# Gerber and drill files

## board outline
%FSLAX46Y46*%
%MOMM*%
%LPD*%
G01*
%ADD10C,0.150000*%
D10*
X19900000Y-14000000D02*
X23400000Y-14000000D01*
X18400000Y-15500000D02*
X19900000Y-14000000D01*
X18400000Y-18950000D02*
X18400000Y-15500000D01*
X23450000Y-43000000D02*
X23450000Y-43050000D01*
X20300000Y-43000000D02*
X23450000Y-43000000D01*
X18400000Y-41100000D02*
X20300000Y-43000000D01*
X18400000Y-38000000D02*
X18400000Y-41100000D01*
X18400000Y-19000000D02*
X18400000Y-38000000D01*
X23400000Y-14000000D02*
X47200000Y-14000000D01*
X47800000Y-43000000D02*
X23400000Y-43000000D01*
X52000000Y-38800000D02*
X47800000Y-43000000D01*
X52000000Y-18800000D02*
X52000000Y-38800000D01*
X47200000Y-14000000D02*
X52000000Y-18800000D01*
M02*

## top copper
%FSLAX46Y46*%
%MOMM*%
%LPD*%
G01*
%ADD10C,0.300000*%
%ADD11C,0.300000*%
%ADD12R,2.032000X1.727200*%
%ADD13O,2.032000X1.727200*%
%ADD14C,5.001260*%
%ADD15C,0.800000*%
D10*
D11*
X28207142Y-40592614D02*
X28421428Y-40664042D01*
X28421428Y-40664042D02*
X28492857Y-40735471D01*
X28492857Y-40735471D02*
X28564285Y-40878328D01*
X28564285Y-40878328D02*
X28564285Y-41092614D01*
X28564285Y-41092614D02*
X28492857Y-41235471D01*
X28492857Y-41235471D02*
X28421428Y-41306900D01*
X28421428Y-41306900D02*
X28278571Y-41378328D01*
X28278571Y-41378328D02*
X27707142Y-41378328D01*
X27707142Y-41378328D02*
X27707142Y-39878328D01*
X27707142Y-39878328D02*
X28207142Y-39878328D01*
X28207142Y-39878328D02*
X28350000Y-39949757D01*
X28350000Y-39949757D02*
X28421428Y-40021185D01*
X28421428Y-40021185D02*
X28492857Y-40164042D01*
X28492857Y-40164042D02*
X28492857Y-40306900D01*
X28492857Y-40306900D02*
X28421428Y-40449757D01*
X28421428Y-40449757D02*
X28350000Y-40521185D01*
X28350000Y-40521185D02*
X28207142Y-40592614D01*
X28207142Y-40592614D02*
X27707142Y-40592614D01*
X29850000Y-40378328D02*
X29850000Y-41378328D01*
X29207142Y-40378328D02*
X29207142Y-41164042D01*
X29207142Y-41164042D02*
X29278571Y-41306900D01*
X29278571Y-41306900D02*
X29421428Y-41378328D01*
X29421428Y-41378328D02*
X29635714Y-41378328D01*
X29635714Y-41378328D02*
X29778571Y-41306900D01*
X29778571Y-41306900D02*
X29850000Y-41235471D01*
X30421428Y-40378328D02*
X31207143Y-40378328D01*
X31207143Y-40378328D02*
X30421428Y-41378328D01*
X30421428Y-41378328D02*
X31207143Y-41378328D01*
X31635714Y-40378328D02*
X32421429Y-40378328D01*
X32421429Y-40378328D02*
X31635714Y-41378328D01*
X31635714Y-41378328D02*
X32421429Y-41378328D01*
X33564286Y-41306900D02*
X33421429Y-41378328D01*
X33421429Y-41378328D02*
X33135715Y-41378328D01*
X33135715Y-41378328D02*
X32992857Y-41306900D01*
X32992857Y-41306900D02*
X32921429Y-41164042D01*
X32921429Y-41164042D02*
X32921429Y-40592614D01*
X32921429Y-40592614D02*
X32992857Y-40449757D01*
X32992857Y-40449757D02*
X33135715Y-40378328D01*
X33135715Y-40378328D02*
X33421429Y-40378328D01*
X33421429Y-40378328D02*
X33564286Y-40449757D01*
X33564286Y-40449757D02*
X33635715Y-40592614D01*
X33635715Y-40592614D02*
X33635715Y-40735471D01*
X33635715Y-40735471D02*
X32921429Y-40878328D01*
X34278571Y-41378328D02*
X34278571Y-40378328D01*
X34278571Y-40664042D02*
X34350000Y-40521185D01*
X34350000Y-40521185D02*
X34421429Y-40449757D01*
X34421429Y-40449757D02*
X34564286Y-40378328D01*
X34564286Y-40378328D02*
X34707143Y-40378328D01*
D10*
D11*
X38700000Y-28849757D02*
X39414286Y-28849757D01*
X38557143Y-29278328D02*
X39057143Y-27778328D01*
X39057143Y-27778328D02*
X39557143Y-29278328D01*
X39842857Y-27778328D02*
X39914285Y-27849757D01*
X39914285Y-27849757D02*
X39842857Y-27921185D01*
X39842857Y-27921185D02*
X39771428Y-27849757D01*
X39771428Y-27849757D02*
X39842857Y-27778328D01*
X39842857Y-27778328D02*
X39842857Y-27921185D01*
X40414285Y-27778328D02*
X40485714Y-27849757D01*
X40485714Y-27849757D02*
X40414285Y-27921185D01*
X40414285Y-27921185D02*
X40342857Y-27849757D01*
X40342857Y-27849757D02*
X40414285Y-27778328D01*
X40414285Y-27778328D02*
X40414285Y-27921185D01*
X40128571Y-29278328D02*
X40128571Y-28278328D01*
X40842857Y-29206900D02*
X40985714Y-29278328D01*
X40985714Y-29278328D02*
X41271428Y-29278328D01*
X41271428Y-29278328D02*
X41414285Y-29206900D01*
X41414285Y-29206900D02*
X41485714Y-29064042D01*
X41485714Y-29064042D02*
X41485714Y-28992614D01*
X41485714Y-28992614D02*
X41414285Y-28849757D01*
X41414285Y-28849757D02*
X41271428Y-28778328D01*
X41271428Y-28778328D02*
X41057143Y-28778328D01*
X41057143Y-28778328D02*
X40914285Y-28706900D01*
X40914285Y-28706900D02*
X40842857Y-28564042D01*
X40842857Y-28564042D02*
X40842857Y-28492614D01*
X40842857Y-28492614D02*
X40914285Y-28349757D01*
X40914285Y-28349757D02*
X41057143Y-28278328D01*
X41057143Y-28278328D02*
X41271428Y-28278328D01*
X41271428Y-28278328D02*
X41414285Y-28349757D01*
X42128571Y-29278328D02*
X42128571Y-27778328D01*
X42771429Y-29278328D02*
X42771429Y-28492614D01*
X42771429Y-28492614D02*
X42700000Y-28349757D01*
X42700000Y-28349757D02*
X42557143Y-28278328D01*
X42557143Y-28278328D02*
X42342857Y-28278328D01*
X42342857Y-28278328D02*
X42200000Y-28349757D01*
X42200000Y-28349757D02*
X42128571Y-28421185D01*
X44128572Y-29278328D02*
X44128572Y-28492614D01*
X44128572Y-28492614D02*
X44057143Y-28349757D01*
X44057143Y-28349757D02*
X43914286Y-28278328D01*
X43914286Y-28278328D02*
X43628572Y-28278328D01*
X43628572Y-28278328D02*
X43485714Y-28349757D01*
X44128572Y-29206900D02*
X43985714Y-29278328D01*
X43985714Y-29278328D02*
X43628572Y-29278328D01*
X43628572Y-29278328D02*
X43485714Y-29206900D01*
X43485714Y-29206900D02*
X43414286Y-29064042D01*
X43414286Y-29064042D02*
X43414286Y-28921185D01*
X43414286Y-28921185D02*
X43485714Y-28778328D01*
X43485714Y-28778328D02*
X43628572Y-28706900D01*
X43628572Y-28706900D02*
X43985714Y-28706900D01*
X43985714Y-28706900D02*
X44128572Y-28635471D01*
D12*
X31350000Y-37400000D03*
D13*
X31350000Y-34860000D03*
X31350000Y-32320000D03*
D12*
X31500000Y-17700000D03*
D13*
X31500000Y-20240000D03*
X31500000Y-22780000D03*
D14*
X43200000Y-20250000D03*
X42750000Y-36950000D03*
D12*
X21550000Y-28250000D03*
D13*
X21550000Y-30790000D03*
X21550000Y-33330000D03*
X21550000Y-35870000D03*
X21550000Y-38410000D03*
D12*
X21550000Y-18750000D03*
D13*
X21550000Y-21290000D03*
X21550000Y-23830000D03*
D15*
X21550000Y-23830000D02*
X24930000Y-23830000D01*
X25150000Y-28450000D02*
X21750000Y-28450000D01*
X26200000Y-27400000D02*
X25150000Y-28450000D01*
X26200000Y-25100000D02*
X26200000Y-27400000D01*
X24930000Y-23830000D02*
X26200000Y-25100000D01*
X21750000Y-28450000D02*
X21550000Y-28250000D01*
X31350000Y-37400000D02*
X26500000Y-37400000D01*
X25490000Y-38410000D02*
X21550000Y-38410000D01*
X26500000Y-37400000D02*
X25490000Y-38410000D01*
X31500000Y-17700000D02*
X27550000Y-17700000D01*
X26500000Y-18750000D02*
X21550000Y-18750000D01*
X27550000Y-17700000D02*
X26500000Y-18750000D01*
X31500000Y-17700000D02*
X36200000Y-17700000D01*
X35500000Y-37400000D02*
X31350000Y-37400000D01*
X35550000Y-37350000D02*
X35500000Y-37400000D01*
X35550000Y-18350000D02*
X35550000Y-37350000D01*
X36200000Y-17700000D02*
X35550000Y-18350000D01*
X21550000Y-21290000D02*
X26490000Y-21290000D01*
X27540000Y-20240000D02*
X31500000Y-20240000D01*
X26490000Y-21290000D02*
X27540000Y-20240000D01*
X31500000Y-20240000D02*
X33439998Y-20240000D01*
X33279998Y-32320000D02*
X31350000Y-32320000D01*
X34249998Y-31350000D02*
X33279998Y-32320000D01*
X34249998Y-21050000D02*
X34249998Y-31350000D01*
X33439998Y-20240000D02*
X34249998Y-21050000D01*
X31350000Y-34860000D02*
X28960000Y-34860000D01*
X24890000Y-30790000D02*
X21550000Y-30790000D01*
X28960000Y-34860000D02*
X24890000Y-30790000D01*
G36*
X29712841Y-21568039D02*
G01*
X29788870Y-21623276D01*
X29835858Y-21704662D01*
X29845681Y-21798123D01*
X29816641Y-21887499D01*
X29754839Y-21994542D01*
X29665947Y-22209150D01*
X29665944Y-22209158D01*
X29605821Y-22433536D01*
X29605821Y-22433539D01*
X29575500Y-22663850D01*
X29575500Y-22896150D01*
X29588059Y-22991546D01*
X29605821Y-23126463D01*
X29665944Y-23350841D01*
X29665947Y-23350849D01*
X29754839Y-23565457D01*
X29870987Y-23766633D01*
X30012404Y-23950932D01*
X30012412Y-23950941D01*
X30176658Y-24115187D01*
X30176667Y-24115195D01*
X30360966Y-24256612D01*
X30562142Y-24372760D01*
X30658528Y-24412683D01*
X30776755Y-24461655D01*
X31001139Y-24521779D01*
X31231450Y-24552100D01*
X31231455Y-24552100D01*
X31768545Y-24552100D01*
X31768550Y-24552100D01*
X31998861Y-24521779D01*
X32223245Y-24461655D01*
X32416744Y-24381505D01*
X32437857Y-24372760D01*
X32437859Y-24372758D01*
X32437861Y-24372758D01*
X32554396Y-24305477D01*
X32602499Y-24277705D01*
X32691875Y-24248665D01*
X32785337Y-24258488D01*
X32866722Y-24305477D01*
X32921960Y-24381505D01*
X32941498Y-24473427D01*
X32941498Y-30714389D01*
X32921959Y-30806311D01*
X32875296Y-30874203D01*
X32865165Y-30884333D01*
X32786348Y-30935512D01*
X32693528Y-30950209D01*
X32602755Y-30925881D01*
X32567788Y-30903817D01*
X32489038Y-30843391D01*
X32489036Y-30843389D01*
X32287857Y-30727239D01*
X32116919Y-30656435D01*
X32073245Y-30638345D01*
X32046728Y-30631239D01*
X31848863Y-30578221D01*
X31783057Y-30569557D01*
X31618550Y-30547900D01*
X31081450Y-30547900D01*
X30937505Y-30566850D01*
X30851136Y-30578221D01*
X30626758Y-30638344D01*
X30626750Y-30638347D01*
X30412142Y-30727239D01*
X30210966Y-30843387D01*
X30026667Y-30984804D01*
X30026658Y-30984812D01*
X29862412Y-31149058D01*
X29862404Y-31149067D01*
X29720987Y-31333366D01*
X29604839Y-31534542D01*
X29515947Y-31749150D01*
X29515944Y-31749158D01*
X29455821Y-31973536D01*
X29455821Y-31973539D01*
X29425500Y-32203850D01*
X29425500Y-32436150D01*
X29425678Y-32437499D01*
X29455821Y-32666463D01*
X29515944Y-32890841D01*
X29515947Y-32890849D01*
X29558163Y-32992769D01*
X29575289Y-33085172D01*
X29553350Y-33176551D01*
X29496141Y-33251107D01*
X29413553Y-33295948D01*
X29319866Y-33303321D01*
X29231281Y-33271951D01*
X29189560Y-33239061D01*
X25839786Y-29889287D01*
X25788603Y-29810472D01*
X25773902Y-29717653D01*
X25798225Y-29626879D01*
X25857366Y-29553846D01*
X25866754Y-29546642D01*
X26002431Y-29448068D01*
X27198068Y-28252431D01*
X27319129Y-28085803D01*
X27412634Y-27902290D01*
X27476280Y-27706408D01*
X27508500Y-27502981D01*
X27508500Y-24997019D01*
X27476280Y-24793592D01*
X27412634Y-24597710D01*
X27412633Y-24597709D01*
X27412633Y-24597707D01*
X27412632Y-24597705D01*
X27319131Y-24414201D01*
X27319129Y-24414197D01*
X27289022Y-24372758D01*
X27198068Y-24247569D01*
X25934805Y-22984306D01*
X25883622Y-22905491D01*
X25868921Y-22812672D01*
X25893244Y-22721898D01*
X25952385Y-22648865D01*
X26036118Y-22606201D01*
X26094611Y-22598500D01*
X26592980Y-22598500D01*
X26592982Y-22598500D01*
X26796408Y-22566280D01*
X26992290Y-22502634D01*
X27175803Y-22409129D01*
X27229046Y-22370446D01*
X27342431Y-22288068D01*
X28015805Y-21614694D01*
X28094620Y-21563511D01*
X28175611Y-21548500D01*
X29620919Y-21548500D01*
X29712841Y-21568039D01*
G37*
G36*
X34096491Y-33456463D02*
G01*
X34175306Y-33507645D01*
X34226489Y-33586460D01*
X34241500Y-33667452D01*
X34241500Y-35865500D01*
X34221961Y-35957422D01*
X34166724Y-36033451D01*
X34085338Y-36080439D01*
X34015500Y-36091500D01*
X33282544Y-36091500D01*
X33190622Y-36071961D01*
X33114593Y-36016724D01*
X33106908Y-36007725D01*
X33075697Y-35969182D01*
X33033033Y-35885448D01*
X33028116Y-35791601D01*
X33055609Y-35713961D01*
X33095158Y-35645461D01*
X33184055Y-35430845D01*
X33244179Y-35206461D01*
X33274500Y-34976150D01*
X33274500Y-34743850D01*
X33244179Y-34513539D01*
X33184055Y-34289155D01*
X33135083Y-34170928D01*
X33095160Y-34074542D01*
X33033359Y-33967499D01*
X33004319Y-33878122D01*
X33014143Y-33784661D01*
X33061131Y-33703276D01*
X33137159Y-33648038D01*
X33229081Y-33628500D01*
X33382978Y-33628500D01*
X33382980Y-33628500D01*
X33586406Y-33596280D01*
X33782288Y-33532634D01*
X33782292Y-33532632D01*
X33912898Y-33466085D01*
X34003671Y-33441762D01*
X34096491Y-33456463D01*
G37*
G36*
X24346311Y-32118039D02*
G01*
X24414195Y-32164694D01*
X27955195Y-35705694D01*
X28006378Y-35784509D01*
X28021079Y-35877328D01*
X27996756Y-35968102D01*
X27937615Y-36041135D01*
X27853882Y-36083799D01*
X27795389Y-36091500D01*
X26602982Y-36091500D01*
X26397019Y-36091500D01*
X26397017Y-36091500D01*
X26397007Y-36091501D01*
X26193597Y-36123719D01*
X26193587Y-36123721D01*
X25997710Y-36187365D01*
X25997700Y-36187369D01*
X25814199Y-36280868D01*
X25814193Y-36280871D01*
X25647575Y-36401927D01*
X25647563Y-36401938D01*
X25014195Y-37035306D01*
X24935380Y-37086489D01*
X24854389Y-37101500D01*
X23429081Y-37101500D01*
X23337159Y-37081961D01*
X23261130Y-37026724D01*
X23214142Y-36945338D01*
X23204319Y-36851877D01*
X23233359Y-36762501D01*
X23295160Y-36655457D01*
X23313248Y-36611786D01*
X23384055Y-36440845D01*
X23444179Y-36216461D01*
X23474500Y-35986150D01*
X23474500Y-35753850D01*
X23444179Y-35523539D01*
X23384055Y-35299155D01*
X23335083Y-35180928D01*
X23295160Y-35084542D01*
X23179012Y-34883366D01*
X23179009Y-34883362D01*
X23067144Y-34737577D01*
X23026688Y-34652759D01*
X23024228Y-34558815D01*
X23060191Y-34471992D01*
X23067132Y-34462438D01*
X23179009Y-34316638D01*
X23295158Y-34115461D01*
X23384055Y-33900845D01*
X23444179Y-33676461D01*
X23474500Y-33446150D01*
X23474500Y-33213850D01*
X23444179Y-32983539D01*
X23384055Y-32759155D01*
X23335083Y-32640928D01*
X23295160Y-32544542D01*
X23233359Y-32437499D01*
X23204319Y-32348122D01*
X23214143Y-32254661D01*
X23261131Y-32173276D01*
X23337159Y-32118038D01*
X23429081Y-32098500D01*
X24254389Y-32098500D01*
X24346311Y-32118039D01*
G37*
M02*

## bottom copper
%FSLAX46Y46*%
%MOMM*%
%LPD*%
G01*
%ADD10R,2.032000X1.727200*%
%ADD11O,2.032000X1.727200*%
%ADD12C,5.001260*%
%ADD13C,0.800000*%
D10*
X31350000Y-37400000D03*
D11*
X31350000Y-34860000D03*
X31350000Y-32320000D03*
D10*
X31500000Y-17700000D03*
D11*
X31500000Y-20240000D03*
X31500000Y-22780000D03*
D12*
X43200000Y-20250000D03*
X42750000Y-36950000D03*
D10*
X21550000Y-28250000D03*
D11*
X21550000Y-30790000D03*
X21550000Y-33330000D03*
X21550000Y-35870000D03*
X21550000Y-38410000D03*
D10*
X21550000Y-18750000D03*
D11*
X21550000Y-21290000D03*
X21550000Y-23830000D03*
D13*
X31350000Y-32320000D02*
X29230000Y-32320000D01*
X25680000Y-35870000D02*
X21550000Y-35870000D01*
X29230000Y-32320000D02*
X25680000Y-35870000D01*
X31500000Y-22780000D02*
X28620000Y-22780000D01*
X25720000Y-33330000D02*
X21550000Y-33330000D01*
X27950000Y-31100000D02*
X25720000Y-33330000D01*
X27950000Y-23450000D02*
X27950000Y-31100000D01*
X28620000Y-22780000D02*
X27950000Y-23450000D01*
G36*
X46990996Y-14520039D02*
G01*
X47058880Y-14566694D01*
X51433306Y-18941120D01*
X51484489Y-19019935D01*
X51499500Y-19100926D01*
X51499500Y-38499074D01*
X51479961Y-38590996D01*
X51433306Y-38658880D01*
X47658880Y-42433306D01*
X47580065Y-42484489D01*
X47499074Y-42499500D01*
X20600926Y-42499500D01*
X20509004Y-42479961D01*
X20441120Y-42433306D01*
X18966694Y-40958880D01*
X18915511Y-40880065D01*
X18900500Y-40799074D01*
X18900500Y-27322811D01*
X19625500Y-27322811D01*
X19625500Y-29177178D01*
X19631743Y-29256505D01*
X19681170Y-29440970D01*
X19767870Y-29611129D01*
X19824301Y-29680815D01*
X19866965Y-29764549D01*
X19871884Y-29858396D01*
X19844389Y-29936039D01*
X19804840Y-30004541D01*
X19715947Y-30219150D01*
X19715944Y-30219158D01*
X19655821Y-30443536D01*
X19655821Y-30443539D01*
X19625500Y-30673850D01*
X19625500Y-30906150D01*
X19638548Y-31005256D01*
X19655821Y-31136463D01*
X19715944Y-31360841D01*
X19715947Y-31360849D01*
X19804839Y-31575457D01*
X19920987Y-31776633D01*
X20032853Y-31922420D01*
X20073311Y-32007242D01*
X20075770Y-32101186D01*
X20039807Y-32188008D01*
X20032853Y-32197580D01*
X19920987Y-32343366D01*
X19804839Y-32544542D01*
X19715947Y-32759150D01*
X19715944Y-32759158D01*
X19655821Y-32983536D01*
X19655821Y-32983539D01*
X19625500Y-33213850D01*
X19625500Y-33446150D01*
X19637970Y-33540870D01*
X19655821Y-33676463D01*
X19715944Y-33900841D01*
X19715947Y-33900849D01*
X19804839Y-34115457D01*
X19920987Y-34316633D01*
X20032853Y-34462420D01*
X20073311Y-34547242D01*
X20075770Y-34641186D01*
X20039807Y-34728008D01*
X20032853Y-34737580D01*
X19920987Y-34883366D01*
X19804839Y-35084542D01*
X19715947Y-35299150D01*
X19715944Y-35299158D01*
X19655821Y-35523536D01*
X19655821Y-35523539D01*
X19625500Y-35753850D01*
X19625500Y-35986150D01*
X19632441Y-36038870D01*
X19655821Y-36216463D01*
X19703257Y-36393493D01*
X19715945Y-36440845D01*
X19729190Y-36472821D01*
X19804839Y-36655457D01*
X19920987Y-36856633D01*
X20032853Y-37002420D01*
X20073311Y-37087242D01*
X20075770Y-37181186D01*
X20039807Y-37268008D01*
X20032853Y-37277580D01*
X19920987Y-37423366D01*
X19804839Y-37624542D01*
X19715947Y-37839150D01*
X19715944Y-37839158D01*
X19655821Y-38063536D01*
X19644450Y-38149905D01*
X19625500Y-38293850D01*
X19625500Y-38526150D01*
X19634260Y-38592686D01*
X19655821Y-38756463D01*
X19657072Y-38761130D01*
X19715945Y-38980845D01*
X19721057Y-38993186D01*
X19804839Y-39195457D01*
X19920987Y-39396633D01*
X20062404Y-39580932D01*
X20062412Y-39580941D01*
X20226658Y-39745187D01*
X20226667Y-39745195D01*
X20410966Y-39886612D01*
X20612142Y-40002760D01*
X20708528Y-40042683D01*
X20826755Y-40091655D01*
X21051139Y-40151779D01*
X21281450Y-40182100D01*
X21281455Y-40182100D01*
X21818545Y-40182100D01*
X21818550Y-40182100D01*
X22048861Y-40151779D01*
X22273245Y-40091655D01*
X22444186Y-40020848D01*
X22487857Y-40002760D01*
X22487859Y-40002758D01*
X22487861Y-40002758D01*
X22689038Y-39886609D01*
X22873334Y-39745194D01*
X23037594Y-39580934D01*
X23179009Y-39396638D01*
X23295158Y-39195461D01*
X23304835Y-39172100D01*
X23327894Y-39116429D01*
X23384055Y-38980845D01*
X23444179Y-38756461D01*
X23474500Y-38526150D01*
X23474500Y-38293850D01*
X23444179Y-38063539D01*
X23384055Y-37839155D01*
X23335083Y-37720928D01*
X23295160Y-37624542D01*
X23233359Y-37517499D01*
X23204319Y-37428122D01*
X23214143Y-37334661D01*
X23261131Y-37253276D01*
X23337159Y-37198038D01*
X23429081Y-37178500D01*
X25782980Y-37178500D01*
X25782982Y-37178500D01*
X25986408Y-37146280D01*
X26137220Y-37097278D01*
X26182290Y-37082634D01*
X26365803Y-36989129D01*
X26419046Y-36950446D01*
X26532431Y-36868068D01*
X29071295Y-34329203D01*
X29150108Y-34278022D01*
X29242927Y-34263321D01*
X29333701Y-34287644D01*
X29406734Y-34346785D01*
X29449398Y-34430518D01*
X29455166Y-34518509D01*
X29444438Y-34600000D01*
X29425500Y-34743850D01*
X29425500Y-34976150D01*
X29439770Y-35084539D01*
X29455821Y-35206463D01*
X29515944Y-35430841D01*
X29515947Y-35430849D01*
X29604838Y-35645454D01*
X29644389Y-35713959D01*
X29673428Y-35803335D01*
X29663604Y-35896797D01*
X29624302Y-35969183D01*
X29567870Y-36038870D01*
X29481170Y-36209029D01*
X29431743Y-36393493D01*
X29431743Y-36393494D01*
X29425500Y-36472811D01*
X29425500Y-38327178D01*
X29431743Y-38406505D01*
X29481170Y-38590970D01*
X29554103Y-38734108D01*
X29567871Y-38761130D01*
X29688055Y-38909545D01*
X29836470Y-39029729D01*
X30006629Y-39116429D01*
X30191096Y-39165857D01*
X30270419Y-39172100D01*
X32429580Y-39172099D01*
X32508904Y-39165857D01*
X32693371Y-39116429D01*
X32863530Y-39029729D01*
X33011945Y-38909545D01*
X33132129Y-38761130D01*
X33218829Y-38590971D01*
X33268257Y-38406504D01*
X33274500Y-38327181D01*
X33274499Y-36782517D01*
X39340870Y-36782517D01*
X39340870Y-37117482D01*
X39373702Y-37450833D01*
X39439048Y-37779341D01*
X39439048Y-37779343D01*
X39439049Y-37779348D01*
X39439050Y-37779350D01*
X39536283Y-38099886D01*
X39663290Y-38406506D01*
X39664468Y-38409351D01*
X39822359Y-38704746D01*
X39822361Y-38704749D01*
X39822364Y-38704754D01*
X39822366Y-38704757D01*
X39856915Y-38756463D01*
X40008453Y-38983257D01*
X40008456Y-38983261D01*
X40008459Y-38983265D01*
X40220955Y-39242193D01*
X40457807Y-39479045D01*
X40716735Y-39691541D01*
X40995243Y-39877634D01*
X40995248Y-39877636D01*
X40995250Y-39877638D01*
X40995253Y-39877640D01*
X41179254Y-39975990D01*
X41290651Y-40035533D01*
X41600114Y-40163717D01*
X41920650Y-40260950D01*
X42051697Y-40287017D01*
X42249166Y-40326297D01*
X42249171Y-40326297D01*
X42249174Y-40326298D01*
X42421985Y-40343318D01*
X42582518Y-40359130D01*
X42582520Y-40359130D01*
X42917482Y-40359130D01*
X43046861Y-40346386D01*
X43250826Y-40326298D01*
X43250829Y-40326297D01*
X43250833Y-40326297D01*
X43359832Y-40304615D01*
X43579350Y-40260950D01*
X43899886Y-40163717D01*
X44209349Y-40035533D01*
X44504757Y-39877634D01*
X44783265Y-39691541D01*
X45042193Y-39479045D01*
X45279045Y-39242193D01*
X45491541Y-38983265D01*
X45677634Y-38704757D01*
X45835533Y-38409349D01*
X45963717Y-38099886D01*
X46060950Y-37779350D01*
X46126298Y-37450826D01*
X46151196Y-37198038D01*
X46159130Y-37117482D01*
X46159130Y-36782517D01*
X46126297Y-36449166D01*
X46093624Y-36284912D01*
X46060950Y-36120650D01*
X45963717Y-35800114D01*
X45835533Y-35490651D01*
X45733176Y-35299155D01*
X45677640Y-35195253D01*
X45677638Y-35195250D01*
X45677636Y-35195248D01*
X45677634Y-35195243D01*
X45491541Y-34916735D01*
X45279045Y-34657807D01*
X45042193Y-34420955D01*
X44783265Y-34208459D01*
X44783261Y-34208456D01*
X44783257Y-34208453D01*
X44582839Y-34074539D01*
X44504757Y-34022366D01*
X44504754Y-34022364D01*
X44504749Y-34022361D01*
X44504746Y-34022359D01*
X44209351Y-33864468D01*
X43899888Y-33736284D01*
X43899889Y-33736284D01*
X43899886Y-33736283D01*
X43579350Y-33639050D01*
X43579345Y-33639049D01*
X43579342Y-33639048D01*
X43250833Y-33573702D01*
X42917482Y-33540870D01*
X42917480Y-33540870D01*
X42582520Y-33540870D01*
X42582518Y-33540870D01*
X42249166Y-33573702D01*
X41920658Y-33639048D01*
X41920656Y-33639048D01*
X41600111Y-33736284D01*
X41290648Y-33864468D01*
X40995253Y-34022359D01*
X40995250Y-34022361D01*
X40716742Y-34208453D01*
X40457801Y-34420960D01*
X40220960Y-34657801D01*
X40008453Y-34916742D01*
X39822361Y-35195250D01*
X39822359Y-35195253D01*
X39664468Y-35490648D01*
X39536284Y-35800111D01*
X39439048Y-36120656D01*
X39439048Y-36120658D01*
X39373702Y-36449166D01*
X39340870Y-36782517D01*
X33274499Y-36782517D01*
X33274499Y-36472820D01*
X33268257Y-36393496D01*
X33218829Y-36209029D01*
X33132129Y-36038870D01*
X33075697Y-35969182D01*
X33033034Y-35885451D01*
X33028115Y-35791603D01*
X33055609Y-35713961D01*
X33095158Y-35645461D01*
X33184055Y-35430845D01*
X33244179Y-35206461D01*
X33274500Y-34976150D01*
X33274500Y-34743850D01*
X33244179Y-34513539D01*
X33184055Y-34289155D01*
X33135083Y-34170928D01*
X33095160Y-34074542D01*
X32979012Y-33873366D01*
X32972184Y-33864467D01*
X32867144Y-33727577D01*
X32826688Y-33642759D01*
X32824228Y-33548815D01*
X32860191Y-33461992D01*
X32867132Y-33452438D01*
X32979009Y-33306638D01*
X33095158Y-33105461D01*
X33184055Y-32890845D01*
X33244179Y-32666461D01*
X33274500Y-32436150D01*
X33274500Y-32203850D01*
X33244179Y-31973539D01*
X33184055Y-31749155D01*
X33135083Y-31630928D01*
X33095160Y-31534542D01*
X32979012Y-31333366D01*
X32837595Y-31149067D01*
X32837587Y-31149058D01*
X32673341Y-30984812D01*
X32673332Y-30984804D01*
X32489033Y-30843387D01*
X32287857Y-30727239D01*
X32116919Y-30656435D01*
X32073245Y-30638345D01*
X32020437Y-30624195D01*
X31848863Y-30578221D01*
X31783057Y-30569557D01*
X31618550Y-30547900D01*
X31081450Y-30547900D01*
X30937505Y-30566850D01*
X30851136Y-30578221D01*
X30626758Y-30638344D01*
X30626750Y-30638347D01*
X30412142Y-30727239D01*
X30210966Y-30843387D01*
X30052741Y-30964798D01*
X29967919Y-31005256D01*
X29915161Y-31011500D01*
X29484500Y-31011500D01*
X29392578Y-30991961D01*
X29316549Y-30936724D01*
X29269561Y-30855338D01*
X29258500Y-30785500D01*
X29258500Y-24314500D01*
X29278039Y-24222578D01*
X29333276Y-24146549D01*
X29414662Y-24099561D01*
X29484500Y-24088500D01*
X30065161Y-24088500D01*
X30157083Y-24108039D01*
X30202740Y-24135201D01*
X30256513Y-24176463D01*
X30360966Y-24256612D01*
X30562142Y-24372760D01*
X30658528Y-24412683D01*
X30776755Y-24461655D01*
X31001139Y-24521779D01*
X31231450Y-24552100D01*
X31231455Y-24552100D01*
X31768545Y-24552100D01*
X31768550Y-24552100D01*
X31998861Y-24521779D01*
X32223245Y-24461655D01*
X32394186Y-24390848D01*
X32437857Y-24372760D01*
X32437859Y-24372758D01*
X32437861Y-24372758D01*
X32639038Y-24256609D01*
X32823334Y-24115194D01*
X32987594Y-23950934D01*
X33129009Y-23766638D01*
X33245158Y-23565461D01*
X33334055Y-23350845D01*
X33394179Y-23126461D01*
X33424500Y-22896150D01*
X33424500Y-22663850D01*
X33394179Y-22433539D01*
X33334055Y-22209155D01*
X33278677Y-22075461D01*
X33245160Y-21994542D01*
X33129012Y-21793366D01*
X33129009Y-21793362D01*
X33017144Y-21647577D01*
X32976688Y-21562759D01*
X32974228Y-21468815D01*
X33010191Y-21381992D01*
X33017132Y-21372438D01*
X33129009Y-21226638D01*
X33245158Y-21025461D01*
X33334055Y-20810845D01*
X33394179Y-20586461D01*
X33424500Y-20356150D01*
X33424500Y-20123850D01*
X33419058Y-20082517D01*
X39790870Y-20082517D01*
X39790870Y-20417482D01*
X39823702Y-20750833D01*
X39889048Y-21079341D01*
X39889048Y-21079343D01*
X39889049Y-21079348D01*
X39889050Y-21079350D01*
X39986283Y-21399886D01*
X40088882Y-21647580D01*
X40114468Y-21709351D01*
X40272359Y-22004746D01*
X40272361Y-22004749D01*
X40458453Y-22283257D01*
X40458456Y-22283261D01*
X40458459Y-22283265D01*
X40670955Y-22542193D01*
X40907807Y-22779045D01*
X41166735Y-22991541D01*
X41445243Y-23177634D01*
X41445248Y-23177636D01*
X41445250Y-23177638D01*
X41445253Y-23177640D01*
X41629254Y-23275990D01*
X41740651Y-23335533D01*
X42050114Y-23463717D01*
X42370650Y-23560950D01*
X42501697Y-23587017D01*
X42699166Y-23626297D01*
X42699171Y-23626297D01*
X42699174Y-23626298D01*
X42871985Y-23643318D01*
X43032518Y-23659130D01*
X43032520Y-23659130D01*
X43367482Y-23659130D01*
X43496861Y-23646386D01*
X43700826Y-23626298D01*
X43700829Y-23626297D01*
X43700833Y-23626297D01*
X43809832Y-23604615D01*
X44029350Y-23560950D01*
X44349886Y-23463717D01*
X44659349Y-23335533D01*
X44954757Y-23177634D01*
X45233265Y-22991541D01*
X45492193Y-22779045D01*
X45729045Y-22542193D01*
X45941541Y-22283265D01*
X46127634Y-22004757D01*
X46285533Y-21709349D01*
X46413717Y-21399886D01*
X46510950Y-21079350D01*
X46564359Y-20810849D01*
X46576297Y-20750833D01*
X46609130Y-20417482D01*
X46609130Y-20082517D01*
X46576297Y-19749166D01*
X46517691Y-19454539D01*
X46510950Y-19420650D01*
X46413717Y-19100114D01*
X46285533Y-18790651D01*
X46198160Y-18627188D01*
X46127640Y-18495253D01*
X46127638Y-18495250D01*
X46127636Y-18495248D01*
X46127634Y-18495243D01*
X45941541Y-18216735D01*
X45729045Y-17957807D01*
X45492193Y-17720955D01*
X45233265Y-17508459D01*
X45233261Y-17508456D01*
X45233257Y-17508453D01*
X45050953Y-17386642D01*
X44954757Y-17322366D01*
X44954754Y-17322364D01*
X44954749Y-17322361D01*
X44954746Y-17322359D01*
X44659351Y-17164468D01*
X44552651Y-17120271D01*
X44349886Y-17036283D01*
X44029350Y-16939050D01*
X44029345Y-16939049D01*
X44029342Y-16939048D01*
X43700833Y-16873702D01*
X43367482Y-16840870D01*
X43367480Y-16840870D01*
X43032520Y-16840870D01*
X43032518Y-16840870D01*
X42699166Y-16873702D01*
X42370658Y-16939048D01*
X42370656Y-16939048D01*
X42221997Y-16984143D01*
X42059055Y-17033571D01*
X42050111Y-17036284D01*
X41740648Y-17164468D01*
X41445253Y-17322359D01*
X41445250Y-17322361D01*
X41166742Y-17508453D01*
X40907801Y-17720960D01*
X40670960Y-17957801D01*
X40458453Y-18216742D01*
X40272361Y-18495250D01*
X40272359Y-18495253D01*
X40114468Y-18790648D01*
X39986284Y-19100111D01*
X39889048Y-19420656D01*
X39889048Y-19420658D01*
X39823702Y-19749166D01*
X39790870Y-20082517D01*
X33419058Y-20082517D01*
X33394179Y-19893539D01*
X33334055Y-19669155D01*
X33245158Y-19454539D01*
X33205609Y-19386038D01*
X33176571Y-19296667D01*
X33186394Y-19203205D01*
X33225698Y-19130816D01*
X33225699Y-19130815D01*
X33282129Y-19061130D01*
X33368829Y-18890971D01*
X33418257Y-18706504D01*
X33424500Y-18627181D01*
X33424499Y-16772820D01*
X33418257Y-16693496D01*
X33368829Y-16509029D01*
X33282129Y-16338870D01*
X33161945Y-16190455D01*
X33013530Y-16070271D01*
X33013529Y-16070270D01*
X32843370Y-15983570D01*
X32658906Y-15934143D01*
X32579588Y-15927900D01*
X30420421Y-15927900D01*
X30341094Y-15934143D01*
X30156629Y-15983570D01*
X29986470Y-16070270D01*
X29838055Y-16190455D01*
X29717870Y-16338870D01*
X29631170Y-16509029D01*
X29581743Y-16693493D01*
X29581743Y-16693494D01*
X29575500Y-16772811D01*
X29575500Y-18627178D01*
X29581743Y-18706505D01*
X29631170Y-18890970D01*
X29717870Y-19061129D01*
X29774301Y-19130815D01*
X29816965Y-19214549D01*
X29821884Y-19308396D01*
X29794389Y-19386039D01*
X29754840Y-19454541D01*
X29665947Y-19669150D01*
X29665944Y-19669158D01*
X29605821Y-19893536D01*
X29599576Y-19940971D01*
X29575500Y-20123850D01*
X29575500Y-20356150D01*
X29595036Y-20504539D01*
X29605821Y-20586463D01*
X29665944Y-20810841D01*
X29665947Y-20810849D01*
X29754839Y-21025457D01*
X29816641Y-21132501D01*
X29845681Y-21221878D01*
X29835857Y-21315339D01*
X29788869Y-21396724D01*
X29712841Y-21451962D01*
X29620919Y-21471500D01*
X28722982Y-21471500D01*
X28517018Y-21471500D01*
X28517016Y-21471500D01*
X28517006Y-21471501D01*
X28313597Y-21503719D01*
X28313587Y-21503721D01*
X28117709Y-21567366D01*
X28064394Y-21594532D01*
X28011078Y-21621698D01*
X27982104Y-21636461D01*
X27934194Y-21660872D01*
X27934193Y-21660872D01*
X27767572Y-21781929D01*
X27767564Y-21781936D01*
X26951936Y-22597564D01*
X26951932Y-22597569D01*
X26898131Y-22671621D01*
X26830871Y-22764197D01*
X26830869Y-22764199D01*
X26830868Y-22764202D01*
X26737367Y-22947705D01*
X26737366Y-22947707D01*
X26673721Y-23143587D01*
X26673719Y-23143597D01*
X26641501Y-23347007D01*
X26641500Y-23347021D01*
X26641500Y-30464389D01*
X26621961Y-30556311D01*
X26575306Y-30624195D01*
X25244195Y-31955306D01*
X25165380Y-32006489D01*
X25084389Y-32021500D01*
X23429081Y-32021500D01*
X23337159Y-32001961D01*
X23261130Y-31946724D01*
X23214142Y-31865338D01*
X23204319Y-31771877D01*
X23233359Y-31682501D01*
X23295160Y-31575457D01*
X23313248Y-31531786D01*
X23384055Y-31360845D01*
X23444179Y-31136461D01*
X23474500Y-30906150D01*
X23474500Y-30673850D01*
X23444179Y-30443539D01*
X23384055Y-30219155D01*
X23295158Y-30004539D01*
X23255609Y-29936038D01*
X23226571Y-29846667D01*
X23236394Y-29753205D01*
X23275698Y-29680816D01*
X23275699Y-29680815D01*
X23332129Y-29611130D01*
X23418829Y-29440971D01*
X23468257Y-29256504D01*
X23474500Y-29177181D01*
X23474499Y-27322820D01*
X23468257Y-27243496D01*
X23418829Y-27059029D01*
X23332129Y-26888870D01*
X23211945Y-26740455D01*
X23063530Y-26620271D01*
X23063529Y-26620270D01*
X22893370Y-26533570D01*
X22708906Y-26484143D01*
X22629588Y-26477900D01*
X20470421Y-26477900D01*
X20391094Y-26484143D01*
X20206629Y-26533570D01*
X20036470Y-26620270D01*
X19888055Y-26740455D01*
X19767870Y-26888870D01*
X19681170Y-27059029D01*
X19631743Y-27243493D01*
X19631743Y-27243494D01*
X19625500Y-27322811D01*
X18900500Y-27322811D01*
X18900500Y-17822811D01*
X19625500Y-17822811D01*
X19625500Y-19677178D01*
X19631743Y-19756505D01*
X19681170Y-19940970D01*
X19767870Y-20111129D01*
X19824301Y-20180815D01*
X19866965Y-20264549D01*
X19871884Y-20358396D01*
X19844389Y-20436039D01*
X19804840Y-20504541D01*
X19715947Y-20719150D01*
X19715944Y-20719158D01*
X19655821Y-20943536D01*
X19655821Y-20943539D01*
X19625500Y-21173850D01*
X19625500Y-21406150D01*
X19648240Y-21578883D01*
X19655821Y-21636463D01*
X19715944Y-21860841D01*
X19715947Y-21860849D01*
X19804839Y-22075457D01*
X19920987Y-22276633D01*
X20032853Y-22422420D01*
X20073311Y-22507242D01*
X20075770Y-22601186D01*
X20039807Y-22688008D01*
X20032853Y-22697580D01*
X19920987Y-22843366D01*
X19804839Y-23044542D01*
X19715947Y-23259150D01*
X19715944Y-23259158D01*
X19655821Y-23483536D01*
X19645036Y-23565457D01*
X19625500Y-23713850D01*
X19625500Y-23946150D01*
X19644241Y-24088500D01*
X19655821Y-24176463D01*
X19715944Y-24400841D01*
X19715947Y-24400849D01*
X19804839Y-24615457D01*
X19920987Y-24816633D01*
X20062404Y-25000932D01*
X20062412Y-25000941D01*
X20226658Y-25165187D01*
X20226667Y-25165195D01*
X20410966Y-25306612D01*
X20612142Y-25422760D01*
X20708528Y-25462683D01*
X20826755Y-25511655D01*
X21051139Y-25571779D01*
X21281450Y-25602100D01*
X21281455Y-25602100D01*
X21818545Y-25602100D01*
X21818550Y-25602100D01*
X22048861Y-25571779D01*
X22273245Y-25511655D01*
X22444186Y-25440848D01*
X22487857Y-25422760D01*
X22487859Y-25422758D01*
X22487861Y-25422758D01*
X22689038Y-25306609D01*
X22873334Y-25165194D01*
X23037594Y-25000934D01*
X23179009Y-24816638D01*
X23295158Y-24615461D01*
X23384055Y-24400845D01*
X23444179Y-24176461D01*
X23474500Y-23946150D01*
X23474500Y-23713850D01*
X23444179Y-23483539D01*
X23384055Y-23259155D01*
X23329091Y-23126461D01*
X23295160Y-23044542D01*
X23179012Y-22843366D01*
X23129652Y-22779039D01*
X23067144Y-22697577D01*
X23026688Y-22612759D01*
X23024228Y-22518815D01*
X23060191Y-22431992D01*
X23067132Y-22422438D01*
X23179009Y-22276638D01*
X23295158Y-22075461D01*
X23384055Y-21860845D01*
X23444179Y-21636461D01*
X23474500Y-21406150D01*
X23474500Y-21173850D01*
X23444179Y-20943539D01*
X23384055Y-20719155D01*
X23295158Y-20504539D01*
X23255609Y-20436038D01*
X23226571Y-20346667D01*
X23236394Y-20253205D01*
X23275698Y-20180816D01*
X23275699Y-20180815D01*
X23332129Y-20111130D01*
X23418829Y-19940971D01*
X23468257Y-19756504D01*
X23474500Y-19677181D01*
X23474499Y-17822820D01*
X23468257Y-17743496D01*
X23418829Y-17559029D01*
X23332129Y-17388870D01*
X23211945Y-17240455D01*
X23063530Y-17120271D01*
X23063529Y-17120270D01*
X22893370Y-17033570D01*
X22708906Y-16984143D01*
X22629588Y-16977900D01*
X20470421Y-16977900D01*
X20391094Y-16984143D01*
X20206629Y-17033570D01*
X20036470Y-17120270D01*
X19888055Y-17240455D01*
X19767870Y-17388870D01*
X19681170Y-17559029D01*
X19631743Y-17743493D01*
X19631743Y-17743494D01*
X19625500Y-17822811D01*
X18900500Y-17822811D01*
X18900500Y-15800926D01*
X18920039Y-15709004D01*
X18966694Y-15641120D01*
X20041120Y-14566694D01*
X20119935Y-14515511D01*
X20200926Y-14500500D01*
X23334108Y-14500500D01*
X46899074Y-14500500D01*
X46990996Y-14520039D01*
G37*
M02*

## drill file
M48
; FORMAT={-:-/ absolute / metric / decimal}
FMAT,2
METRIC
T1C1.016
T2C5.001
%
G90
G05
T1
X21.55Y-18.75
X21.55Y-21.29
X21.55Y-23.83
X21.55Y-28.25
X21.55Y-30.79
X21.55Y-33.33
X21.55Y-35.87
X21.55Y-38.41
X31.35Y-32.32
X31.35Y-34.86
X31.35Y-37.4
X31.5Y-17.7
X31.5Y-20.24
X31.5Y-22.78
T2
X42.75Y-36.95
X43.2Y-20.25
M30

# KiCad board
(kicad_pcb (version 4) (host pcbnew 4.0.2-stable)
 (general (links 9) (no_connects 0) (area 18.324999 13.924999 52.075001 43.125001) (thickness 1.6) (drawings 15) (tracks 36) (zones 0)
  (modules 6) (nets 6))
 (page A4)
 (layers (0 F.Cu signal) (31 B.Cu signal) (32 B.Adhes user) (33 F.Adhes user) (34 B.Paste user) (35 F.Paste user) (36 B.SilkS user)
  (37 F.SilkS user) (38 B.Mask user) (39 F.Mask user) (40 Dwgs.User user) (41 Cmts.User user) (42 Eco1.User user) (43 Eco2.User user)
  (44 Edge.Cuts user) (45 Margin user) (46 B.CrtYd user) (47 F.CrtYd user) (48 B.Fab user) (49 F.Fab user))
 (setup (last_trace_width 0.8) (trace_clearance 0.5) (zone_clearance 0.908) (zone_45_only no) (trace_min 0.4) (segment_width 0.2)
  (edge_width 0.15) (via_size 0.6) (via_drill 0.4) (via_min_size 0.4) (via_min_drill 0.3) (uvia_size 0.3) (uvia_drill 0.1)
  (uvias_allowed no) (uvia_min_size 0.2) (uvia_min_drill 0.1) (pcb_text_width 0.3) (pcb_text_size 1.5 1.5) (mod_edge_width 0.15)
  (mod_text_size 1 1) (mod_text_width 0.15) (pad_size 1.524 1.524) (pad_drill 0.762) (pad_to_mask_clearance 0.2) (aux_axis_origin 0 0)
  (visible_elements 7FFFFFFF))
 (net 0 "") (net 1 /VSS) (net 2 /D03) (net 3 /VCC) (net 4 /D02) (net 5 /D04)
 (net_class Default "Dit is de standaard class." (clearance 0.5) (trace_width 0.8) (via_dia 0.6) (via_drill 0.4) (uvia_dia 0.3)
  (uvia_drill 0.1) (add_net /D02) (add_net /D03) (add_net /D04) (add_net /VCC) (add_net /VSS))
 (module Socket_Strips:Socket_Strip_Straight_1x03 (layer F.Cu) (at 31.35 37.4 90)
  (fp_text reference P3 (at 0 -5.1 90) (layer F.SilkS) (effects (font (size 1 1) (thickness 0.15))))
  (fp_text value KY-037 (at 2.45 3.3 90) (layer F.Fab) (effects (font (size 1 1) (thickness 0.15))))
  (pad 1 thru_hole rect (at 0 0 90) (size 1.7272 2.032) (drill 1.016) (layers *.Cu *.Mask F.SilkS) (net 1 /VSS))
  (pad 2 thru_hole oval (at 2.54 0 90) (size 1.7272 2.032) (drill 1.016) (layers *.Cu *.Mask F.SilkS) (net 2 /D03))
  (pad 3 thru_hole oval (at 5.08 0 90) (size 1.7272 2.032) (drill 1.016) (layers *.Cu *.Mask F.SilkS) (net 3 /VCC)))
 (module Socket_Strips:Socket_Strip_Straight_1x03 (layer F.Cu) (at 31.5 17.7 270)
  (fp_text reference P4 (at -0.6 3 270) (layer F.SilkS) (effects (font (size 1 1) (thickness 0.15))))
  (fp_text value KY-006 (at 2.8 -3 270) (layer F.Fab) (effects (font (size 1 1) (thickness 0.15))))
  (pad 1 thru_hole rect (at 0 0 270) (size 1.7272 2.032) (drill 1.016) (layers *.Cu *.Mask F.SilkS) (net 1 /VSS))
  (pad 2 thru_hole oval (at 2.54 0 270) (size 1.7272 2.032) (drill 1.016) (layers *.Cu *.Mask F.SilkS) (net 3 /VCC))
  (pad 3 thru_hole oval (at 5.08 0 270) (size 1.7272 2.032) (drill 1.016) (layers *.Cu *.Mask F.SilkS) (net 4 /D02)))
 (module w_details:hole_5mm (layer F.Cu) (at 43.2 20.25)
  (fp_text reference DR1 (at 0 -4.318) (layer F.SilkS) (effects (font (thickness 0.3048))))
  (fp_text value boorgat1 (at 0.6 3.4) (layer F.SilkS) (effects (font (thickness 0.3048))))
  (pad 1 thru_hole circle (at 0 0) (size 5.00126 5.00126) (drill 5.00126) (layers *.Cu F.SilkS)))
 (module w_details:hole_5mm (layer F.Cu) (at 42.75 36.95)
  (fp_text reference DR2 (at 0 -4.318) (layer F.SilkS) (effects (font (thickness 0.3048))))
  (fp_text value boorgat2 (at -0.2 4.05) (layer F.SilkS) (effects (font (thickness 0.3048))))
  (pad 1 thru_hole circle (at 0 0) (size 5.00126 5.00126) (drill 5.00126) (layers *.Cu F.SilkS)))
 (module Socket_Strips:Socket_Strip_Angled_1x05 (layer F.Cu) (at 21.55 28.25 270)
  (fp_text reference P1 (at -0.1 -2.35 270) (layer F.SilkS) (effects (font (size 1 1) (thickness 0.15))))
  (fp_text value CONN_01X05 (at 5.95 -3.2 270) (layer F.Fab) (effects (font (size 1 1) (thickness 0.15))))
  (pad 1 thru_hole rect (at 0 0 270) (size 1.7272 2.032) (drill 1.016) (layers *.Cu *.Mask F.SilkS) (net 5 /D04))
  (pad 2 thru_hole oval (at 2.54 0 270) (size 1.7272 2.032) (drill 1.016) (layers *.Cu *.Mask F.SilkS) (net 2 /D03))
  (pad 3 thru_hole oval (at 5.08 0 270) (size 1.7272 2.032) (drill 1.016) (layers *.Cu *.Mask F.SilkS) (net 4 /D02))
  (pad 4 thru_hole oval (at 7.62 0 270) (size 1.7272 2.032) (drill 1.016) (layers *.Cu *.Mask F.SilkS) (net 3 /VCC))
  (pad 5 thru_hole oval (at 10.16 0 270) (size 1.7272 2.032) (drill 1.016) (layers *.Cu *.Mask F.SilkS) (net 1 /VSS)))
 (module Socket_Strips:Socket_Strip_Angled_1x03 (layer F.Cu) (at 21.55 18.75 270)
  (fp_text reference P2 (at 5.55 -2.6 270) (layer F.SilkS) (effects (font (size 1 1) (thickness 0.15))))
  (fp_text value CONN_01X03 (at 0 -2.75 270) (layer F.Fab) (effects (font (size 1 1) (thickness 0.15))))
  (pad 1 thru_hole rect (at 0 0 270) (size 1.7272 2.032) (drill 1.016) (layers *.Cu *.Mask F.SilkS) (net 1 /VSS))
  (pad 2 thru_hole oval (at 2.54 0 270) (size 1.7272 2.032) (drill 1.016) (layers *.Cu *.Mask F.SilkS) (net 3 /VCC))
  (pad 3 thru_hole oval (at 5.08 0 270) (size 1.7272 2.032) (drill 1.016) (layers *.Cu *.Mask F.SilkS) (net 5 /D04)))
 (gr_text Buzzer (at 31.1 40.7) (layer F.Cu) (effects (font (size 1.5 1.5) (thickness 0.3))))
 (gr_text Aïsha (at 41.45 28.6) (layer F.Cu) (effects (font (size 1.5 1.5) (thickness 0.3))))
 (gr_line (start 19.9 14) (end 23.4 14) (angle 90) (layer Edge.Cuts) (width 0.15))
 (gr_line (start 18.4 15.5) (end 19.9 14) (angle 90) (layer Edge.Cuts) (width 0.15))
 (gr_line (start 18.4 18.95) (end 18.4 15.5) (angle 90) (layer Edge.Cuts) (width 0.15))
 (gr_line (start 23.45 43) (end 23.45 43.05) (angle 90) (layer Edge.Cuts) (width 0.15))
 (gr_line (start 20.3 43) (end 23.45 43) (angle 90) (layer Edge.Cuts) (width 0.15))
 (gr_line (start 18.4 41.1) (end 20.3 43) (angle 90) (layer Edge.Cuts) (width 0.15))
 (gr_line (start 18.4 38) (end 18.4 41.1) (angle 90) (layer Edge.Cuts) (width 0.15))
 (gr_line (start 18.4 19) (end 18.4 38) (angle 90) (layer Edge.Cuts) (width 0.15))
 (gr_line (start 23.4 14) (end 47.2 14) (angle 90) (layer Edge.Cuts) (width 0.15))
 (gr_line (start 47.8 43) (end 23.4 43) (angle 90) (layer Edge.Cuts) (width 0.15))
 (gr_line (start 52 38.8) (end 47.8 43) (angle 90) (layer Edge.Cuts) (width 0.15))
 (gr_line (start 52 18.8) (end 52 38.8) (angle 90) (layer Edge.Cuts) (width 0.15))
 (gr_line (start 47.2 14) (end 52 18.8) (angle 90) (layer Edge.Cuts) (width 0.15))
 (segment (start 21.55 23.83) (end 24.93 23.83) (width 0.8) (layer F.Cu) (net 5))
 (segment (start 25.15 28.45) (end 21.75 28.45) (width 0.8) (layer F.Cu) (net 5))
 (segment (start 26.2 27.4) (end 25.15 28.45) (width 0.8) (layer F.Cu) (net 5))
 (segment (start 26.2 25.1) (end 26.2 27.4) (width 0.8) (layer F.Cu) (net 5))
 (segment (start 24.93 23.83) (end 26.2 25.1) (width 0.8) (layer F.Cu) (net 5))
 (segment (start 21.75 28.45) (end 21.55 28.25) (width 0.8) (layer F.Cu) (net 5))
 (segment (start 31.35 37.4) (end 26.5 37.4) (width 0.8) (layer F.Cu) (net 1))
 (segment (start 25.49 38.41) (end 21.55 38.41) (width 0.8) (layer F.Cu) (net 1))
 (segment (start 26.5 37.4) (end 25.49 38.41) (width 0.8) (layer F.Cu) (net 1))
 (segment (start 31.5 17.7) (end 27.55 17.7) (width 0.8) (layer F.Cu) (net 1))
 (segment (start 26.5 18.75) (end 21.55 18.75) (width 0.8) (layer F.Cu) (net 1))
 (segment (start 27.55 17.7) (end 26.5 18.75) (width 0.8) (layer F.Cu) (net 1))
 (segment (start 31.5 17.7) (end 36.2 17.7) (width 0.8) (layer F.Cu) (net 1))
 (segment (start 35.5 37.4) (end 31.35 37.4) (width 0.8) (layer F.Cu) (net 1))
 (segment (start 35.55 37.35) (end 35.5 37.4) (width 0.8) (layer F.Cu) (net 1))
 (segment (start 35.55 18.35) (end 35.55 37.35) (width 0.8) (layer F.Cu) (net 1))
 (segment (start 36.2 17.7) (end 35.55 18.35) (width 0.8) (layer F.Cu) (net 1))
 (segment (start 31.35 32.32) (end 29.23 32.32) (width 0.8) (layer B.Cu) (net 3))
 (segment (start 25.68 35.87) (end 21.55 35.87) (width 0.8) (layer B.Cu) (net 3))
 (segment (start 29.23 32.32) (end 25.68 35.87) (width 0.8) (layer B.Cu) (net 3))
 (segment (start 21.55 21.29) (end 26.49 21.29) (width 0.8) (layer F.Cu) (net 3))
 (segment (start 27.54 20.24) (end 31.5 20.24) (width 0.8) (layer F.Cu) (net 3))
 (segment (start 26.49 21.29) (end 27.54 20.24) (width 0.8) (layer F.Cu) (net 3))
 (segment (start 31.5 20.24) (end 33.439998 20.24) (width 0.8) (layer F.Cu) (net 3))
 (segment (start 33.279998 32.32) (end 31.35 32.32) (width 0.8) (layer F.Cu) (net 3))
 (segment (start 34.249998 31.35) (end 33.279998 32.32) (width 0.8) (layer F.Cu) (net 3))
 (segment (start 34.249998 21.05) (end 34.249998 31.35) (width 0.8) (layer F.Cu) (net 3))
 (segment (start 33.439998 20.24) (end 34.249998 21.05) (width 0.8) (layer F.Cu) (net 3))
 (segment (start 31.35 34.86) (end 28.96 34.86) (width 0.8) (layer F.Cu) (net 2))
 (segment (start 24.89 30.79) (end 21.55 30.79) (width 0.8) (layer F.Cu) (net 2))
 (segment (start 28.96 34.86) (end 24.89 30.79) (width 0.8) (layer F.Cu) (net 2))
 (segment (start 31.5 22.78) (end 28.62 22.78) (width 0.8) (layer B.Cu) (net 4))
 (segment (start 25.72 33.33) (end 21.55 33.33) (width 0.8) (layer B.Cu) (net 4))
 (segment (start 27.95 31.1) (end 25.72 33.33) (width 0.8) (layer B.Cu) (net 4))
 (segment (start 27.95 23.45) (end 27.95 31.1) (width 0.8) (layer B.Cu) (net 4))
 (segment (start 28.62 22.78) (end 27.95 23.45) (width 0.8) (layer B.Cu) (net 4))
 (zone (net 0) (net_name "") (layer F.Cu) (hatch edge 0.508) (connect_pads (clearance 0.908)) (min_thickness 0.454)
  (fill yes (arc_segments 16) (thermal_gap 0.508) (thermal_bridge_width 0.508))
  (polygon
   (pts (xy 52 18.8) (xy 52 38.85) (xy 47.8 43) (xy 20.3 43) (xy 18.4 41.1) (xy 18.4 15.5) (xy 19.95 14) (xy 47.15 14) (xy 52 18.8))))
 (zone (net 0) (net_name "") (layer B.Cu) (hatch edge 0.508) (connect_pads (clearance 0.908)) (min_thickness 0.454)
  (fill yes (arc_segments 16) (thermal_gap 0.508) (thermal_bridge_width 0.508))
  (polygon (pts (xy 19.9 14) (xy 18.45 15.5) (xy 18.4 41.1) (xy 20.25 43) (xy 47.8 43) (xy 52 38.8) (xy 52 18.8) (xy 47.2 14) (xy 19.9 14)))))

